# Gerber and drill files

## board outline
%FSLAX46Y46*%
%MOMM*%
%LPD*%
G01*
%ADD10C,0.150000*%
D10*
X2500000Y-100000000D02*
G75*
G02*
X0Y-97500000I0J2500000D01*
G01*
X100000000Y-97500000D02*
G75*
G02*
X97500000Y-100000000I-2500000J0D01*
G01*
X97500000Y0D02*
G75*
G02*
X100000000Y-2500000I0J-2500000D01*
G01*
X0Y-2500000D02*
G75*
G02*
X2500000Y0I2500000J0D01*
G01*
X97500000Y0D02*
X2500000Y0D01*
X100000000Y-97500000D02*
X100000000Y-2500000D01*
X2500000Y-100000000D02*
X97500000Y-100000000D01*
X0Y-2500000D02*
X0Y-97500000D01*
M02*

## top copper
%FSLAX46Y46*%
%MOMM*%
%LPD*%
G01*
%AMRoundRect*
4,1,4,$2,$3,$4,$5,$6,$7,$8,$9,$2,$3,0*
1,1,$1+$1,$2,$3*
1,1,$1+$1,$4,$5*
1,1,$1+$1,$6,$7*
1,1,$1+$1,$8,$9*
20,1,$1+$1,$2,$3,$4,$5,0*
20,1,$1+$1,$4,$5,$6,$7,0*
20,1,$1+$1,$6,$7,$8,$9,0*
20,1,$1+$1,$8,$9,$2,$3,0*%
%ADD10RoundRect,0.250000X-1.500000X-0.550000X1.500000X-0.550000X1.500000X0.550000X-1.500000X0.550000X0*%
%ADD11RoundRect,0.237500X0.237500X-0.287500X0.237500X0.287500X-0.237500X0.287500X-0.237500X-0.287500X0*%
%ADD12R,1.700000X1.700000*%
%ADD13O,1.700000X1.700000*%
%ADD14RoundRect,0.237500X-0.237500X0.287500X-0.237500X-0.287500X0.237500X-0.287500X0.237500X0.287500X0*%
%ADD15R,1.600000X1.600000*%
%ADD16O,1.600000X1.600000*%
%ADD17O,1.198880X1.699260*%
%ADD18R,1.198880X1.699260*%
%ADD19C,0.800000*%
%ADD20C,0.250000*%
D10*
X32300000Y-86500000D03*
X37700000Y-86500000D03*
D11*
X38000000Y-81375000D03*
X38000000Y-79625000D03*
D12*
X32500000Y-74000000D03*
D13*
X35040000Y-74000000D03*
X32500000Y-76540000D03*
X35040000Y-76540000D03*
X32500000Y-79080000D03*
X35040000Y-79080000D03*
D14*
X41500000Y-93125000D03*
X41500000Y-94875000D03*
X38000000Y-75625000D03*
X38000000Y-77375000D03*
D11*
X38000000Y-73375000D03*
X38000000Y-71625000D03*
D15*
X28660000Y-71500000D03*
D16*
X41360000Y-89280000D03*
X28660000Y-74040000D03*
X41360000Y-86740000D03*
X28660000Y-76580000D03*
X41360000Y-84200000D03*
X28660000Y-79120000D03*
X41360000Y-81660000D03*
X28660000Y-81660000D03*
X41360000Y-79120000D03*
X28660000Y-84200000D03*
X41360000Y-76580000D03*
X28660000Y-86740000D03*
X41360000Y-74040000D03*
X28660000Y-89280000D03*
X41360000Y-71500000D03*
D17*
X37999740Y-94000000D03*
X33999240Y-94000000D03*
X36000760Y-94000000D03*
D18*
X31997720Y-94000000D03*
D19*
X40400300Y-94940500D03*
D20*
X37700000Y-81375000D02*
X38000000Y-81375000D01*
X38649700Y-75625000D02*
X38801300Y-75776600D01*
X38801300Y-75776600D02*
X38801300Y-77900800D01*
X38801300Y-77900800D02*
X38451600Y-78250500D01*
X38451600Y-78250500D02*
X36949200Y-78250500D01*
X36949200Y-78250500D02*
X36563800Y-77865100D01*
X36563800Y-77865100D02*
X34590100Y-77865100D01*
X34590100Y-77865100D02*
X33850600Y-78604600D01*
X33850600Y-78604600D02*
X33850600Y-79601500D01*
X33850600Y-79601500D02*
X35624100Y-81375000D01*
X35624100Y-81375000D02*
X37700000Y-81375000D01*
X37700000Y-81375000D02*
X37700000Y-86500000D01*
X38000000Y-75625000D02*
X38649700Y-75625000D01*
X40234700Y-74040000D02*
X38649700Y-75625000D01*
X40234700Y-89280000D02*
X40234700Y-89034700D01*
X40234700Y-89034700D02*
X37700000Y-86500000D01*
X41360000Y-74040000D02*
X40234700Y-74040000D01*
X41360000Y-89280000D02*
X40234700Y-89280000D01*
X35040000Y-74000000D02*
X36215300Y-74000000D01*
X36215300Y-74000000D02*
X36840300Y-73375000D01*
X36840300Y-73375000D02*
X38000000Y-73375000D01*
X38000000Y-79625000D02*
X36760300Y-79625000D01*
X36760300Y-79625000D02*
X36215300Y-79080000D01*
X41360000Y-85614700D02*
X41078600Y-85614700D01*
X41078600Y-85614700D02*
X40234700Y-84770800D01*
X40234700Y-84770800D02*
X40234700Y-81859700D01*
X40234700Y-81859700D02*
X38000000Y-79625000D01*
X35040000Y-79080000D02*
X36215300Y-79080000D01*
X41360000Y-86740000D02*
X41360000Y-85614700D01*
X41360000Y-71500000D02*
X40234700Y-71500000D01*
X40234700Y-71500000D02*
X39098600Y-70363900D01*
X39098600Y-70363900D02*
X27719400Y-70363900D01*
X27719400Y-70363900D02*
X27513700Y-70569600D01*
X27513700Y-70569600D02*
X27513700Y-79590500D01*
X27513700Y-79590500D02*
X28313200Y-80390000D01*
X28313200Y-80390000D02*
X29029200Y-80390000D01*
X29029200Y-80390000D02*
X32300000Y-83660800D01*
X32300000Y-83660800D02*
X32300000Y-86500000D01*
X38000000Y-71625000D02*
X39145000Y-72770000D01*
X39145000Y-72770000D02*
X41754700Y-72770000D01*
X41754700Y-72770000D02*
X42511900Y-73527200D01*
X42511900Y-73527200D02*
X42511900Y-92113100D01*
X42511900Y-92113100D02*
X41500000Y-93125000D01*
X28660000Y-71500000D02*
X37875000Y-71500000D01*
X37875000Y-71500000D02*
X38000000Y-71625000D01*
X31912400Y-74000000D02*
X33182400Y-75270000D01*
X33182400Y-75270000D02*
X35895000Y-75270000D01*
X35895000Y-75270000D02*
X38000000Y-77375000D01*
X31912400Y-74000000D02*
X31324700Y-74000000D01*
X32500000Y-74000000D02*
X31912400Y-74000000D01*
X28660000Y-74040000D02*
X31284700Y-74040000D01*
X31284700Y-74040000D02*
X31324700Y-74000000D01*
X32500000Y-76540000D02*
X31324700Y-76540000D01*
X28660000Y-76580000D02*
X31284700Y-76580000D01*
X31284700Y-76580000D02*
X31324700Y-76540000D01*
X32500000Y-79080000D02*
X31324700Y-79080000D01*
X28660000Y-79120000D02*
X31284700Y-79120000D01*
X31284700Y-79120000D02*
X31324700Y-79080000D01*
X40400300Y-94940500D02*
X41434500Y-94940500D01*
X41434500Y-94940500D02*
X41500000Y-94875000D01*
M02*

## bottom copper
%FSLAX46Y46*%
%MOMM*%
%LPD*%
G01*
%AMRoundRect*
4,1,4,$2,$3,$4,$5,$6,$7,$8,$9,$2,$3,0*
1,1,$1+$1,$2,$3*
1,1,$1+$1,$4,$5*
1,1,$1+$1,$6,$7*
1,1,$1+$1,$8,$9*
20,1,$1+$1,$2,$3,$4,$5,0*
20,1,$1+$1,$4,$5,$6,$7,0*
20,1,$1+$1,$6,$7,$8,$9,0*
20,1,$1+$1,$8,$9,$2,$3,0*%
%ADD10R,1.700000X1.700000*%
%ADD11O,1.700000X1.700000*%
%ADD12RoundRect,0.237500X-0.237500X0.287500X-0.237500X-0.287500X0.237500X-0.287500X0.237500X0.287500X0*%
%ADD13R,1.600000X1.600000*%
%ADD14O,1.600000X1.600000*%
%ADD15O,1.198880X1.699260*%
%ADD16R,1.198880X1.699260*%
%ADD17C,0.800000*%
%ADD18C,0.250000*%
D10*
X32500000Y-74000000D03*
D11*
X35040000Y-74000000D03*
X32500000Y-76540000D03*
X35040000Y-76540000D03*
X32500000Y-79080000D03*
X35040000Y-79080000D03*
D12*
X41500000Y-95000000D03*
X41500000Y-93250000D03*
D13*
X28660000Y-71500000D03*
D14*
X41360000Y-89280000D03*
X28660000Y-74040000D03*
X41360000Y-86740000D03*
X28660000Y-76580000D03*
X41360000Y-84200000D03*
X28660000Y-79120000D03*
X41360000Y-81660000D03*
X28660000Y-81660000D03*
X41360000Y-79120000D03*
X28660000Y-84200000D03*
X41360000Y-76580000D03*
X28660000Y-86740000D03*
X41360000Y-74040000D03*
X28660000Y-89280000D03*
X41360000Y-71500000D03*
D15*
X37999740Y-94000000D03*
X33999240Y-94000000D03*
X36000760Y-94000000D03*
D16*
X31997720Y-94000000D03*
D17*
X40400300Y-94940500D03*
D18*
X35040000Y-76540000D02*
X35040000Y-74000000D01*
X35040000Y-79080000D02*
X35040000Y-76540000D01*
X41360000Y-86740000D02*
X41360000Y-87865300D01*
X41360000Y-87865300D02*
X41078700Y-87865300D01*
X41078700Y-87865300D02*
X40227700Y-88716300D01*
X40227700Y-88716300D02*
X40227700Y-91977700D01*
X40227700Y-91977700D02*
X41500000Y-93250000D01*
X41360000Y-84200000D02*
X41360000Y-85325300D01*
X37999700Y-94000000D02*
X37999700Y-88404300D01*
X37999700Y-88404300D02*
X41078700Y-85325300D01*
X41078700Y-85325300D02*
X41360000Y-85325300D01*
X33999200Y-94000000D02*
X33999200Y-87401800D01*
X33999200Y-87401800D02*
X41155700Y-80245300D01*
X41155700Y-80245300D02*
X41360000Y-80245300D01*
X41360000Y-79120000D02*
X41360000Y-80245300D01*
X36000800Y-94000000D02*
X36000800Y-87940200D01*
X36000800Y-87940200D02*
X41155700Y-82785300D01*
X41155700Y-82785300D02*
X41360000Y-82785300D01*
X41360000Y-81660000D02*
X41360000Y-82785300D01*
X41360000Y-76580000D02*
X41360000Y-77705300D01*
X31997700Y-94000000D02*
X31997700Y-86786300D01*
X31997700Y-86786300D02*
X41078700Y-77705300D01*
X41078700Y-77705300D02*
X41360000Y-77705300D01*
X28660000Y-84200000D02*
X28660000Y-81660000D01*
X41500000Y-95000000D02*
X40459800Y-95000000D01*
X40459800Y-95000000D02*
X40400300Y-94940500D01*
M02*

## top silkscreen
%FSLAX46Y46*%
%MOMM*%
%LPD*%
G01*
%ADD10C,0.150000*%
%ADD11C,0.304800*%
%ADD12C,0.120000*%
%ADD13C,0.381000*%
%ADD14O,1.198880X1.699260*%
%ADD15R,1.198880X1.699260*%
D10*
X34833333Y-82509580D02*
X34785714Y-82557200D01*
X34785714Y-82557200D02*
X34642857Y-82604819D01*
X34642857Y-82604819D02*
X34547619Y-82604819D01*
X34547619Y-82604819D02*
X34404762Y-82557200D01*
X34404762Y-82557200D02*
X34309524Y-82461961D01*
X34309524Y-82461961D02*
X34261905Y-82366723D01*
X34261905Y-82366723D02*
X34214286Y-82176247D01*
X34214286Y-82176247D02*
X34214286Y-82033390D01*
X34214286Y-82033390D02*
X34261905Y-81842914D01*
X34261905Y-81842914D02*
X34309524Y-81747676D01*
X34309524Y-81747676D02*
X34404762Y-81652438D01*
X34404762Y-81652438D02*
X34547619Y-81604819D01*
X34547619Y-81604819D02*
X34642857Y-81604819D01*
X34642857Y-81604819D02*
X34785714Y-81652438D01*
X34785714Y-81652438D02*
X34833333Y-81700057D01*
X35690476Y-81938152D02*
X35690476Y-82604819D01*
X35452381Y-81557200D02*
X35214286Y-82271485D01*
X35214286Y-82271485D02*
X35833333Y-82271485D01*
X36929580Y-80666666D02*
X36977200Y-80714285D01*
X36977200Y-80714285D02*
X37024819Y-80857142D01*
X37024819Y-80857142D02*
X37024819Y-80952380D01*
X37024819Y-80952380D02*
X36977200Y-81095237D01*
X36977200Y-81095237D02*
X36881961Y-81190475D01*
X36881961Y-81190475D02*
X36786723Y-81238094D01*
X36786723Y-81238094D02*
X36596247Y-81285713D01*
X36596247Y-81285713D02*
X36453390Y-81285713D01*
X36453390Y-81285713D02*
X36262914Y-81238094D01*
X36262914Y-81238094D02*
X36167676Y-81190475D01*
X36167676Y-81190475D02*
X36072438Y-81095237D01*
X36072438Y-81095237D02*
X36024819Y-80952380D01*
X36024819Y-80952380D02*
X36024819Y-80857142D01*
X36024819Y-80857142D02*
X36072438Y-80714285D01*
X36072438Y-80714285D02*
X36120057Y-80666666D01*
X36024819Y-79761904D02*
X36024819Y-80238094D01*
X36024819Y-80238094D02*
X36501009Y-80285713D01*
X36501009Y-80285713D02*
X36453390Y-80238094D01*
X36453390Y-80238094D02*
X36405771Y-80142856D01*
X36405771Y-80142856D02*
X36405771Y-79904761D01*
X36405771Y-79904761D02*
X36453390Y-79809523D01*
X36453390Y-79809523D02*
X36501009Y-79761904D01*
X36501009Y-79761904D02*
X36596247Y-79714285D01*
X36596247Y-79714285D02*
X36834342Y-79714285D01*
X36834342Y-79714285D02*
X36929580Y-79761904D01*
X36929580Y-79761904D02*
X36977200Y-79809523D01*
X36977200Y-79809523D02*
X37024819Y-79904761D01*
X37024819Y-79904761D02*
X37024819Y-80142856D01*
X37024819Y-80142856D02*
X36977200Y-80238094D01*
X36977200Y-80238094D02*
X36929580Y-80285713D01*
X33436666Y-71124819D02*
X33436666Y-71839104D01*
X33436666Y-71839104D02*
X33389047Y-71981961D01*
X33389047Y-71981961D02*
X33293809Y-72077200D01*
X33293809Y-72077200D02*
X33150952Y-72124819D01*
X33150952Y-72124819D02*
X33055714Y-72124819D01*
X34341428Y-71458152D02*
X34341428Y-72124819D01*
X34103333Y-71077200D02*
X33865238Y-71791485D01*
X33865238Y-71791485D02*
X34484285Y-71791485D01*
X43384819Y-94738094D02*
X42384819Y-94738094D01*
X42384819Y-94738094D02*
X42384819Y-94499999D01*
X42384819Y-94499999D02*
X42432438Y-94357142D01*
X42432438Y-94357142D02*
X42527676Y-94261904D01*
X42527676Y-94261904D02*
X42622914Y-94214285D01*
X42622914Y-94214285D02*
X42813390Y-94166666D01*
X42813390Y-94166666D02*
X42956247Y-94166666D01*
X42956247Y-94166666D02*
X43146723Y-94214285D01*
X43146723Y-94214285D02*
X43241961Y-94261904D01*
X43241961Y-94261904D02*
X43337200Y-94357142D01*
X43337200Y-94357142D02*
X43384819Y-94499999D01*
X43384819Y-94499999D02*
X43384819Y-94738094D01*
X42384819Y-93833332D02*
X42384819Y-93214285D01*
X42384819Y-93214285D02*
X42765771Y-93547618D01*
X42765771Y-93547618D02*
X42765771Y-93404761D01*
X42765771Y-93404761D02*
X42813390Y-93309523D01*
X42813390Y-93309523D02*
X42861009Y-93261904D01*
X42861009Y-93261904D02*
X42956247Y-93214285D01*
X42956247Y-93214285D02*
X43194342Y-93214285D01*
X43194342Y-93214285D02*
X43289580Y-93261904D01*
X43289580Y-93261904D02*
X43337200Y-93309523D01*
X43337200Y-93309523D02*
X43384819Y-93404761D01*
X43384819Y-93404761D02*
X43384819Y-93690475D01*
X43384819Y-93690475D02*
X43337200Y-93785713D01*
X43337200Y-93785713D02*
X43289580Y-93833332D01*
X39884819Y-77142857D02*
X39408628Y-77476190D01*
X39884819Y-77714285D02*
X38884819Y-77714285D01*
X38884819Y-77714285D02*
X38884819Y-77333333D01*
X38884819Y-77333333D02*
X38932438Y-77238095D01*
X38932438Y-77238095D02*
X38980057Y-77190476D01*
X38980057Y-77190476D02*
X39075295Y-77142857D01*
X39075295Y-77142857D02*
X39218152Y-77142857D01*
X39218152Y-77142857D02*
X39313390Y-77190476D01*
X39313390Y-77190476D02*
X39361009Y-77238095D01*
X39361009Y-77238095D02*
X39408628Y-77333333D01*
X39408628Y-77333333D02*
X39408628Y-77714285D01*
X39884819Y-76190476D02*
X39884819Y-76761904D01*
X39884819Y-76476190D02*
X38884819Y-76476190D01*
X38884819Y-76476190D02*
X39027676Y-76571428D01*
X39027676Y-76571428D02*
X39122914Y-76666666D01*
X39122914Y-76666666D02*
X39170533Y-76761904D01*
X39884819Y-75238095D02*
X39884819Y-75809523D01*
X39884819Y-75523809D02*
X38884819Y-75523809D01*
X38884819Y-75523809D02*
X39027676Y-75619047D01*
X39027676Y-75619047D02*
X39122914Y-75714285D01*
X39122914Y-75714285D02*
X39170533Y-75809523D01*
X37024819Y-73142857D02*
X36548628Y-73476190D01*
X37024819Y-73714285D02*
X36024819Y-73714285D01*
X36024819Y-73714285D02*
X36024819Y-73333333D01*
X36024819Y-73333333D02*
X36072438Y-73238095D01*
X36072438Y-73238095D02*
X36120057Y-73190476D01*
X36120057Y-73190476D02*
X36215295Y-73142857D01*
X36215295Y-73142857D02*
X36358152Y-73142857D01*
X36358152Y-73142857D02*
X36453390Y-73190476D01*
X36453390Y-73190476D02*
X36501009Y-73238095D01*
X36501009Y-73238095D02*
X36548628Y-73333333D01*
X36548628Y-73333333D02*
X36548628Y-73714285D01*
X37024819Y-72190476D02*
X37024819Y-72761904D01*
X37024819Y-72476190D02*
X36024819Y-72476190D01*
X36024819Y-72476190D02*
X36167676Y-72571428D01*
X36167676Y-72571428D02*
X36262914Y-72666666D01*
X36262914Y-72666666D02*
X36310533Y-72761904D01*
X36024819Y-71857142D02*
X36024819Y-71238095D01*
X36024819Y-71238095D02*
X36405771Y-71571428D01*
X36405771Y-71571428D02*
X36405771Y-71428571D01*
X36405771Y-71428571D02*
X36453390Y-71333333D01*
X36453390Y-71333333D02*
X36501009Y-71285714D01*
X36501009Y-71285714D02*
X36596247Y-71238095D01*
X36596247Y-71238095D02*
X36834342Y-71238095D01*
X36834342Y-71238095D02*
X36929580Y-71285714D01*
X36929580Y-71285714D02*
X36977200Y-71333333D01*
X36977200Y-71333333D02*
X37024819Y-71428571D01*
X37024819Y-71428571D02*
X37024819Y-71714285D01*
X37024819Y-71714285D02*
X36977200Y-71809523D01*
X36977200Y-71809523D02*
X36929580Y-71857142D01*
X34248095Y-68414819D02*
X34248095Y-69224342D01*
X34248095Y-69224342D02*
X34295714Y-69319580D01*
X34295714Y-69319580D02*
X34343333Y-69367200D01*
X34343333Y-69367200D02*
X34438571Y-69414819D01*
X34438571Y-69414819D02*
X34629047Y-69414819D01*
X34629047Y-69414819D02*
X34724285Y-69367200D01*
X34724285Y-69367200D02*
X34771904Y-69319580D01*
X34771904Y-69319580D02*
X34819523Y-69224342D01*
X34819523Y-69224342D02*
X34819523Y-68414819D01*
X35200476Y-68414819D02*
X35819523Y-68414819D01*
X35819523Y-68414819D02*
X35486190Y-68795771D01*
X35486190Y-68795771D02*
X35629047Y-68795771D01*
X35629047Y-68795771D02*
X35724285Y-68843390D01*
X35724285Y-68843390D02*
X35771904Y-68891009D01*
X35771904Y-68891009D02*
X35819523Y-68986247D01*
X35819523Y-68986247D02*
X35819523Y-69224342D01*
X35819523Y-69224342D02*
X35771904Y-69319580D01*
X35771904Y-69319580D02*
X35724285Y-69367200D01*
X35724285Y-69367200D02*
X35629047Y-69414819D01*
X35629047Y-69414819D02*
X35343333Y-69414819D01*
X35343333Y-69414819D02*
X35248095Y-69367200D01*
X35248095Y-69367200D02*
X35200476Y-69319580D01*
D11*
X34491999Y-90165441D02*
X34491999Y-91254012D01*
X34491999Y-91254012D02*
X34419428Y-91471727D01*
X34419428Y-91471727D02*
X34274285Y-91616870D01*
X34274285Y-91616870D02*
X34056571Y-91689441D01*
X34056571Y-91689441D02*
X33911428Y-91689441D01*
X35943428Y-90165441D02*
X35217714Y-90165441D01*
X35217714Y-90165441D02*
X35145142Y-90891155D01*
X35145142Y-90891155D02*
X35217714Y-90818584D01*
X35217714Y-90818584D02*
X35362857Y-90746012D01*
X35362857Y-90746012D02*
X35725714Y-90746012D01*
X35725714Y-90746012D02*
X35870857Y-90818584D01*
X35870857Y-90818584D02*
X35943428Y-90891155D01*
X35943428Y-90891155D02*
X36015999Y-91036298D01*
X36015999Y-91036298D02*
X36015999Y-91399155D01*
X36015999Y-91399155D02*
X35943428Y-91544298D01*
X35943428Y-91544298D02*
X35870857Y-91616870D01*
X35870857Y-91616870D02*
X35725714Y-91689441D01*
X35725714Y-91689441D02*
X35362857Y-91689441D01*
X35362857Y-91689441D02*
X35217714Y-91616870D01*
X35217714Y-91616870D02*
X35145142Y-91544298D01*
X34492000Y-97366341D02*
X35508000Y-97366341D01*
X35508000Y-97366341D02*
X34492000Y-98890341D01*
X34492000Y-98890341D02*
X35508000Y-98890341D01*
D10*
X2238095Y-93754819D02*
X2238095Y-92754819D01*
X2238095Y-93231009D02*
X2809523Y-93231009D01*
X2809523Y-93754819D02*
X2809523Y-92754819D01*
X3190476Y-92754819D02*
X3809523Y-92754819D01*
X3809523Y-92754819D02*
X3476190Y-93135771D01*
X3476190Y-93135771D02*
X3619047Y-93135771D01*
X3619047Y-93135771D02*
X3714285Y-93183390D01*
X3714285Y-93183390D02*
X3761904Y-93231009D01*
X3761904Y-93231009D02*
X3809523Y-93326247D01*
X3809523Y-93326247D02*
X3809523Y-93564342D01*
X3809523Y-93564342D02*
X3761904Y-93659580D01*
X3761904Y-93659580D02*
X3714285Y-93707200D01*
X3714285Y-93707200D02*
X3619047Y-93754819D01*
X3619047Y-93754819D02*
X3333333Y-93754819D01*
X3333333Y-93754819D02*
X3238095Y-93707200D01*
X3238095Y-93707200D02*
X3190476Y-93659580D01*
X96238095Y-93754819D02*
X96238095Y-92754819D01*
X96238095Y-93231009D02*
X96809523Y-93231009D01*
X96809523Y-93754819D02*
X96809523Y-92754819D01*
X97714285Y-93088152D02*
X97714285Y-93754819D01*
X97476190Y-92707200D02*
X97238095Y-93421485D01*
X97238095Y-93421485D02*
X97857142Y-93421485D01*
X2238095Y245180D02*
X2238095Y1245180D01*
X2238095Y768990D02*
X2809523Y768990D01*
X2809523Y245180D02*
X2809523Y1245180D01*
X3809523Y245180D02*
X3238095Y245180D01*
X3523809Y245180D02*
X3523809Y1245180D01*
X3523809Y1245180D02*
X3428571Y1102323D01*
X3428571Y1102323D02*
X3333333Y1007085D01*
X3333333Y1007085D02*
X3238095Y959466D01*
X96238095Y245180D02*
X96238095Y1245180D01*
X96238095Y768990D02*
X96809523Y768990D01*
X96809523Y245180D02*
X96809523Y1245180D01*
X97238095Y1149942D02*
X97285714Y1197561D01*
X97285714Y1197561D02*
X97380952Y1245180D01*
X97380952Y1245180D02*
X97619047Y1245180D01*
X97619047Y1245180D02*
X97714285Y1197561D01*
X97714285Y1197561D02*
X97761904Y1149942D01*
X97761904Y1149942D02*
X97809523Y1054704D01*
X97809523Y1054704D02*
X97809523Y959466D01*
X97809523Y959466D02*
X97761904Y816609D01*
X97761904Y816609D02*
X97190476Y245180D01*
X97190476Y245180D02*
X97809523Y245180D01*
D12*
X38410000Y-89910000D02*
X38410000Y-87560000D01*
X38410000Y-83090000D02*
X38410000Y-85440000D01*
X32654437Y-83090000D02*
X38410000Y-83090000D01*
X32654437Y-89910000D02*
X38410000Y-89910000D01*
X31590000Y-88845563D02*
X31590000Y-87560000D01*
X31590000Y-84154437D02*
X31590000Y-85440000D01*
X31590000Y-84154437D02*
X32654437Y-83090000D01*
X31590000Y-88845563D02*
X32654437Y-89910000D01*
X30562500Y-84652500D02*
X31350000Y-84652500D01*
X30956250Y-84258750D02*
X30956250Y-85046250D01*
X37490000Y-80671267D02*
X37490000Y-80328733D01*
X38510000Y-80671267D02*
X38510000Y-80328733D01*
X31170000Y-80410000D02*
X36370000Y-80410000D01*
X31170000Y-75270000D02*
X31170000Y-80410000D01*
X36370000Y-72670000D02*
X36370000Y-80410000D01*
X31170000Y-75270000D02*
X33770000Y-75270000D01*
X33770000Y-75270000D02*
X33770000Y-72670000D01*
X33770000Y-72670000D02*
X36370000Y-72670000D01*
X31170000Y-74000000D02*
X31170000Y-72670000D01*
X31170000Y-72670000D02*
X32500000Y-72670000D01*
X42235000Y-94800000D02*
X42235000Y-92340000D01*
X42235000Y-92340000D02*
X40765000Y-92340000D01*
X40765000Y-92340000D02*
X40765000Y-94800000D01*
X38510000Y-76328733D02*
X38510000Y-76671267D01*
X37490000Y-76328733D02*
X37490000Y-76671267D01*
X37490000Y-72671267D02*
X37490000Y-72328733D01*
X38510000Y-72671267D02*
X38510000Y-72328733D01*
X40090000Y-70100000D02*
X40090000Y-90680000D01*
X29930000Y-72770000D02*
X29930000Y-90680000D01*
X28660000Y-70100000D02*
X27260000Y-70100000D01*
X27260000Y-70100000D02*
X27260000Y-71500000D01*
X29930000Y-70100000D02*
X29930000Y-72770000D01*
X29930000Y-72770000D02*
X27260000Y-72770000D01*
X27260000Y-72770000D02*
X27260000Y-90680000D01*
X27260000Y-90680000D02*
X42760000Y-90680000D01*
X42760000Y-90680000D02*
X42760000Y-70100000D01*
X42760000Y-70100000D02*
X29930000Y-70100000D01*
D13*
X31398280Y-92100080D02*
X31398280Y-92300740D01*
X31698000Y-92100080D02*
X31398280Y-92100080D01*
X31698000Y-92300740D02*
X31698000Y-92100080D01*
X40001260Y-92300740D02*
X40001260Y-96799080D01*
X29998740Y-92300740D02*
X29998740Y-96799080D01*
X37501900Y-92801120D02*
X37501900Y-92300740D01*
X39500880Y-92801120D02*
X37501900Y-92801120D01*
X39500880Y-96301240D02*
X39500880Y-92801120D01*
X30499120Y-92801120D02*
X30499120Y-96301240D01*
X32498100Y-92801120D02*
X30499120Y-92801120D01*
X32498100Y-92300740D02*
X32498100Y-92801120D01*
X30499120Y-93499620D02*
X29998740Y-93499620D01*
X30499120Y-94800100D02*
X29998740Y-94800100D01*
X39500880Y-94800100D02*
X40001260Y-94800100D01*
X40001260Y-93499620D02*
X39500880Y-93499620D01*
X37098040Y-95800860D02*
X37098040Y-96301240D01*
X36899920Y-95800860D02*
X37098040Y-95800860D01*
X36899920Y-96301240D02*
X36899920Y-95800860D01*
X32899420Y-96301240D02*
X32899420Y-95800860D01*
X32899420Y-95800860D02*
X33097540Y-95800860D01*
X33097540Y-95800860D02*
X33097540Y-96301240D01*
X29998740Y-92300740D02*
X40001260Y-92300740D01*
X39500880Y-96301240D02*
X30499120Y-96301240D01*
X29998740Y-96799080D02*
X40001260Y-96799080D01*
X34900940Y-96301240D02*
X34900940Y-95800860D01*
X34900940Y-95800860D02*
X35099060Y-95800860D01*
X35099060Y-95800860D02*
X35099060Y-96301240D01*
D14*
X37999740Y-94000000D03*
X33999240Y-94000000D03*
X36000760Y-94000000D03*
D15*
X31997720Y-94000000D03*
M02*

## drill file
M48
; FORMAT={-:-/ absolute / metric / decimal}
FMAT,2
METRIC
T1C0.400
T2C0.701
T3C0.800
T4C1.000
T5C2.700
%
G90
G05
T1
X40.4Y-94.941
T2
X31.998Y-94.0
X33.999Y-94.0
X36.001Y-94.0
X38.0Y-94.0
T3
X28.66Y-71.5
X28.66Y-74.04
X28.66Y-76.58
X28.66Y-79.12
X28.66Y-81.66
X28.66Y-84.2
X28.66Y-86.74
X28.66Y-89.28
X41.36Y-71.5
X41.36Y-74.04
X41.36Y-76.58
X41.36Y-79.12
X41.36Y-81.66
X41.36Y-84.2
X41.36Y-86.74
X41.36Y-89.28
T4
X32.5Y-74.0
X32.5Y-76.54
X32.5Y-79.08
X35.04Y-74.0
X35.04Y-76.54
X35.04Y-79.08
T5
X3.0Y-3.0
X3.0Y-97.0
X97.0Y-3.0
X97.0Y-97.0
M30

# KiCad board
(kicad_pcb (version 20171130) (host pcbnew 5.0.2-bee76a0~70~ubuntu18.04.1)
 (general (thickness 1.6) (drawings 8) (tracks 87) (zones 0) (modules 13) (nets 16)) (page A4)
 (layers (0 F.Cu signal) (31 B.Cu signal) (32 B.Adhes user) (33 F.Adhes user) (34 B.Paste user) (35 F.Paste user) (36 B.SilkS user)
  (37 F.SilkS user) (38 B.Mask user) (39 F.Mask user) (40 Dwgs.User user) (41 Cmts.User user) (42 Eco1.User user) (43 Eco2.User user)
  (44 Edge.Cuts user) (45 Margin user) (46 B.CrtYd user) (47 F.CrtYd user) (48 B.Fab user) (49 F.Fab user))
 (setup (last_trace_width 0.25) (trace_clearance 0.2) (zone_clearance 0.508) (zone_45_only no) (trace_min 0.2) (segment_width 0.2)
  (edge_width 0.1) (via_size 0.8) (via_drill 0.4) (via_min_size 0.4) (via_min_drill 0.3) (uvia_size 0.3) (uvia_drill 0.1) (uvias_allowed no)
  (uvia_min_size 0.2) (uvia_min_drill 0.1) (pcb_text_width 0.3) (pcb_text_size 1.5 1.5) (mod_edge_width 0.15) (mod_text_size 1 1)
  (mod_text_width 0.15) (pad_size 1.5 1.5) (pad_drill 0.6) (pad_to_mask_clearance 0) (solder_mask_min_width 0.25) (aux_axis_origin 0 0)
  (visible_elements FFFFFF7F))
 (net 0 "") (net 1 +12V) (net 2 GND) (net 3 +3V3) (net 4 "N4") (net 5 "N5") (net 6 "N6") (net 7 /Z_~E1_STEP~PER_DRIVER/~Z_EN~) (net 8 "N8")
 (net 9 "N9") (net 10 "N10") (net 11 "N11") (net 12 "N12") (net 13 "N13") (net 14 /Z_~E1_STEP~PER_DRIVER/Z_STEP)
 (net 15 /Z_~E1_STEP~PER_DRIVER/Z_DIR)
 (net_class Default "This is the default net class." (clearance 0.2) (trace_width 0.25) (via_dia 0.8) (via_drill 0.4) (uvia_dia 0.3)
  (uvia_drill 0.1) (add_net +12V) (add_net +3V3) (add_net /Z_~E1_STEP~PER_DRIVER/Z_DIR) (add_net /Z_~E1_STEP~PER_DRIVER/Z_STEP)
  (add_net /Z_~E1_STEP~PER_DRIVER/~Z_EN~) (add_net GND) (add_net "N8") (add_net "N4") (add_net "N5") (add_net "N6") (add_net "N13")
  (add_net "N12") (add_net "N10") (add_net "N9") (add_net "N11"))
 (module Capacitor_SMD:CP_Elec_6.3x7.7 (layer F.Cu) (at 35 86.5)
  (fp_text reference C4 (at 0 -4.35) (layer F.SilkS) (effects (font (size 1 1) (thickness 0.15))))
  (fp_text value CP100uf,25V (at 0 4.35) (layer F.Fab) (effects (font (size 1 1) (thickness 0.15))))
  (fp_line (start 3.41 3.41) (end 3.41 1.06) (layer F.SilkS) (width 0.12))
  (fp_line (start 3.41 -3.41) (end 3.41 -1.06) (layer F.SilkS) (width 0.12))
  (fp_line (start -2.345563 -3.41) (end 3.41 -3.41) (layer F.SilkS) (width 0.12))
  (fp_line (start -2.345563 3.41) (end 3.41 3.41) (layer F.SilkS) (width 0.12))
  (fp_line (start -3.41 2.345563) (end -3.41 1.06) (layer F.SilkS) (width 0.12))
  (fp_line (start -3.41 -2.345563) (end -3.41 -1.06) (layer F.SilkS) (width 0.12))
  (fp_line (start -3.41 -2.345563) (end -2.345563 -3.41) (layer F.SilkS) (width 0.12))
  (fp_line (start -3.41 2.345563) (end -2.345563 3.41) (layer F.SilkS) (width 0.12))
  (fp_line (start -4.4375 -1.8475) (end -3.65 -1.8475) (layer F.SilkS) (width 0.12))
  (fp_line (start -4.04375 -2.24125) (end -4.04375 -1.45375) (layer F.SilkS) (width 0.12))
  (pad 1 smd roundrect (at -2.7 0) (size 3.5 1.6) (layers F.Cu F.Paste F.Mask) (roundrect_rratio 0.15625) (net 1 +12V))
  (pad 2 smd roundrect (at 2.7 0) (size 3.5 1.6) (layers F.Cu F.Paste F.Mask) (roundrect_rratio 0.15625) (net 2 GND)))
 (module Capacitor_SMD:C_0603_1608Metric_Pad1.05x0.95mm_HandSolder (layer F.Cu) (at 38 80.5 90)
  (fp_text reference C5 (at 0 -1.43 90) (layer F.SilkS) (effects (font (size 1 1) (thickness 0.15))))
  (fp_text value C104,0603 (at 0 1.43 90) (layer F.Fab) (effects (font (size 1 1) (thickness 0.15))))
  (fp_line (start -0.171267 -0.51) (end 0.171267 -0.51) (layer F.SilkS) (width 0.12))
  (fp_line (start -0.171267 0.51) (end 0.171267 0.51) (layer F.SilkS) (width 0.12))
  (pad 1 smd roundrect (at -0.875 0 90) (size 1.05 0.95) (layers F.Cu F.Paste F.Mask) (roundrect_rratio 0.25) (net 2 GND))
  (pad 2 smd roundrect (at 0.875 0 90) (size 1.05 0.95) (layers F.Cu F.Paste F.Mask) (roundrect_rratio 0.25) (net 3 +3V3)))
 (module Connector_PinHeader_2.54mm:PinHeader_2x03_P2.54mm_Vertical (layer F.Cu) (at 32.5 74)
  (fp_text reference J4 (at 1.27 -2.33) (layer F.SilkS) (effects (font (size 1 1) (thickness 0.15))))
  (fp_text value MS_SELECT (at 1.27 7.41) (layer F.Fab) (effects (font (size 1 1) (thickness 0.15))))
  (fp_line (start -1.33 6.41) (end 3.87 6.41) (layer F.SilkS) (width 0.12))
  (fp_line (start -1.33 1.27) (end -1.33 6.41) (layer F.SilkS) (width 0.12))
  (fp_line (start 3.87 -1.33) (end 3.87 6.41) (layer F.SilkS) (width 0.12))
  (fp_line (start -1.33 1.27) (end 1.27 1.27) (layer F.SilkS) (width 0.12))
  (fp_line (start 1.27 1.27) (end 1.27 -1.33) (layer F.SilkS) (width 0.12))
  (fp_line (start 1.27 -1.33) (end 3.87 -1.33) (layer F.SilkS) (width 0.12))
  (fp_line (start -1.33 0) (end -1.33 -1.33) (layer F.SilkS) (width 0.12))
  (fp_line (start -1.33 -1.33) (end 0 -1.33) (layer F.SilkS) (width 0.12))
  (pad 1 thru_hole rect (at 0 0) (size 1.7 1.7) (drill 1) (layers *.Cu *.Mask) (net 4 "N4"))
  (pad 2 thru_hole oval (at 2.54 0) (size 1.7 1.7) (drill 1) (layers *.Cu *.Mask) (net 3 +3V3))
  (pad 3 thru_hole oval (at 0 2.54) (size 1.7 1.7) (drill 1) (layers *.Cu *.Mask) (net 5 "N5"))
  (pad 4 thru_hole oval (at 2.54 2.54) (size 1.7 1.7) (drill 1) (layers *.Cu *.Mask) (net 3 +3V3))
  (pad 5 thru_hole oval (at 0 5.08) (size 1.7 1.7) (drill 1) (layers *.Cu *.Mask) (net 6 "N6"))
  (pad 6 thru_hole oval (at 2.54 5.08) (size 1.7 1.7) (drill 1) (layers *.Cu *.Mask) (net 3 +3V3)))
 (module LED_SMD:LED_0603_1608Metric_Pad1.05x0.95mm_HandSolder (layer F.Cu) (at 41.5 94 270)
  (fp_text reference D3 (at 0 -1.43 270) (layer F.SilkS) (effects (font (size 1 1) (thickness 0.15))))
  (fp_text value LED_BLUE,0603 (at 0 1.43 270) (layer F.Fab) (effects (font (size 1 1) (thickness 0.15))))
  (fp_line (start 0.8 -0.735) (end -1.66 -0.735) (layer F.SilkS) (width 0.12))
  (fp_line (start -1.66 -0.735) (end -1.66 0.735) (layer F.SilkS) (width 0.12))
  (fp_line (start -1.66 0.735) (end 0.8 0.735) (layer F.SilkS) (width 0.12))
  (pad 1 smd roundrect (at -0.875 0 270) (size 1.05 0.95) (layers F.Cu F.Paste F.Mask) (roundrect_rratio 0.25)
   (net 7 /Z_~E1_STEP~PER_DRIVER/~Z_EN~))
  (pad 2 smd roundrect (at 0.875 0 270) (size 1.05 0.95) (layers F.Cu F.Paste F.Mask) (roundrect_rratio 0.25) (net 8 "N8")))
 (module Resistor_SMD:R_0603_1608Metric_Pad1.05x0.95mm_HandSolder (layer F.Cu) (at 38 76.5 270)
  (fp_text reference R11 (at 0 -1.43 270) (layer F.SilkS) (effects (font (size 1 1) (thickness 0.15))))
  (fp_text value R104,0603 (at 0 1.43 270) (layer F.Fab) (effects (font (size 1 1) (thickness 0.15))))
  (fp_line (start -0.171267 -0.51) (end 0.171267 -0.51) (layer F.SilkS) (width 0.12))
  (fp_line (start -0.171267 0.51) (end 0.171267 0.51) (layer F.SilkS) (width 0.12))
  (pad 1 smd roundrect (at -0.875 0 270) (size 1.05 0.95) (layers F.Cu F.Paste F.Mask) (roundrect_rratio 0.25) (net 2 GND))
  (pad 2 smd roundrect (at 0.875 0 270) (size 1.05 0.95) (layers F.Cu F.Paste F.Mask) (roundrect_rratio 0.25) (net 4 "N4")))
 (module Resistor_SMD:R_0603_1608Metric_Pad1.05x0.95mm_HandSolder (layer B.Cu) (at 41.5 94.125 270)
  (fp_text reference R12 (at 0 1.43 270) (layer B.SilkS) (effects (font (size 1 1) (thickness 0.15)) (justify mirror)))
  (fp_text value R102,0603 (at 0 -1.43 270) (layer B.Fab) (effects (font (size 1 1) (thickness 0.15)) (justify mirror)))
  (pad 2 smd roundrect (at 0.875 0 270) (size 1.05 0.95) (layers B.Cu B.Paste B.Mask) (roundrect_rratio 0.25) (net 8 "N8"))
  (pad 1 smd roundrect (at -0.875 0 270) (size 1.05 0.95) (layers B.Cu B.Paste B.Mask) (roundrect_rratio 0.25) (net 3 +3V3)))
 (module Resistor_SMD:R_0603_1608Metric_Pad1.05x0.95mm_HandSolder (layer F.Cu) (at 38 72.5 90)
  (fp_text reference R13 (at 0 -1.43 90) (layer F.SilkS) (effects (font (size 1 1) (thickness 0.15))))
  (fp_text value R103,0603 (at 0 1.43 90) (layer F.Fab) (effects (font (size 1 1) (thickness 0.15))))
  (fp_line (start -0.171267 -0.51) (end 0.171267 -0.51) (layer F.SilkS) (width 0.12))
  (fp_line (start -0.171267 0.51) (end 0.171267 0.51) (layer F.SilkS) (width 0.12))
  (pad 1 smd roundrect (at -0.875 0 90) (size 1.05 0.95) (layers F.Cu F.Paste F.Mask) (roundrect_rratio 0.25) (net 3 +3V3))
  (pad 2 smd roundrect (at 0.875 0 90) (size 1.05 0.95) (layers F.Cu F.Paste F.Mask) (roundrect_rratio 0.25)
   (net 7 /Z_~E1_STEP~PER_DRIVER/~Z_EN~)))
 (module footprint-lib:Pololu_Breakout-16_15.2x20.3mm (layer F.Cu) (at 28.66 71.5)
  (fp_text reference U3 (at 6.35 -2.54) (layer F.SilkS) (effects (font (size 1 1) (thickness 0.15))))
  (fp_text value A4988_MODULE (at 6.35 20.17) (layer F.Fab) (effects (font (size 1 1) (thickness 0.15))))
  (fp_line (start 11.43 -1.4) (end 11.43 19.18) (layer F.SilkS) (width 0.12))
  (fp_line (start 1.27 1.27) (end 1.27 19.18) (layer F.SilkS) (width 0.12))
  (fp_line (start 0 -1.4) (end -1.4 -1.4) (layer F.SilkS) (width 0.12))
  (fp_line (start -1.4 -1.4) (end -1.4 0) (layer F.SilkS) (width 0.12))
  (fp_line (start 1.27 -1.4) (end 1.27 1.27) (layer F.SilkS) (width 0.12))
  (fp_line (start 1.27 1.27) (end -1.4 1.27) (layer F.SilkS) (width 0.12))
  (fp_line (start -1.4 1.27) (end -1.4 19.18) (layer F.SilkS) (width 0.12))
  (fp_line (start -1.4 19.18) (end 14.1 19.18) (layer F.SilkS) (width 0.12))
  (fp_line (start 14.1 19.18) (end 14.1 -1.4) (layer F.SilkS) (width 0.12))
  (fp_line (start 14.1 -1.4) (end 1.27 -1.4) (layer F.SilkS) (width 0.12))
  (pad 1 thru_hole rect (at 0 0) (size 1.6 1.6) (drill 0.8) (layers *.Cu *.Mask) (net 7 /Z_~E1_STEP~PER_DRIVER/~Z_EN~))
  (pad 9 thru_hole oval (at 12.7 17.78) (size 1.6 1.6) (drill 0.8) (layers *.Cu *.Mask) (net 2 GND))
  (pad 2 thru_hole oval (at 0 2.54) (size 1.6 1.6) (drill 0.8) (layers *.Cu *.Mask) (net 4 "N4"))
  (pad 10 thru_hole oval (at 12.7 15.24) (size 1.6 1.6) (drill 0.8) (layers *.Cu *.Mask) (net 3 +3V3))
  (pad 3 thru_hole oval (at 0 5.08) (size 1.6 1.6) (drill 0.8) (layers *.Cu *.Mask) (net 5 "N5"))
  (pad 11 thru_hole oval (at 12.7 12.7) (size 1.6 1.6) (drill 0.8) (layers *.Cu *.Mask) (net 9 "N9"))
  (pad 4 thru_hole oval (at 0 7.62) (size 1.6 1.6) (drill 0.8) (layers *.Cu *.Mask) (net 6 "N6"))
  (pad 12 thru_hole oval (at 12.7 10.16) (size 1.6 1.6) (drill 0.8) (layers *.Cu *.Mask) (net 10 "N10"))
  (pad 5 thru_hole oval (at 0 10.16) (size 1.6 1.6) (drill 0.8) (layers *.Cu *.Mask) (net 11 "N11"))
  (pad 13 thru_hole oval (at 12.7 7.62) (size 1.6 1.6) (drill 0.8) (layers *.Cu *.Mask) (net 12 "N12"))
  (pad 6 thru_hole oval (at 0 12.7) (size 1.6 1.6) (drill 0.8) (layers *.Cu *.Mask) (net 11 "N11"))
  (pad 14 thru_hole oval (at 12.7 5.08) (size 1.6 1.6) (drill 0.8) (layers *.Cu *.Mask) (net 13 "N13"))
  (pad 7 thru_hole oval (at 0 15.24) (size 1.6 1.6) (drill 0.8) (layers *.Cu *.Mask) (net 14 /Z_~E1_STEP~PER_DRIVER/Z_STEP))
  (pad 15 thru_hole oval (at 12.7 2.54) (size 1.6 1.6) (drill 0.8) (layers *.Cu *.Mask) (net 2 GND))
  (pad 8 thru_hole oval (at 0 17.78) (size 1.6 1.6) (drill 0.8) (layers *.Cu *.Mask) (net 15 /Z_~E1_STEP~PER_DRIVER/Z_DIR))
  (pad 16 thru_hole oval (at 12.7 0) (size 1.6 1.6) (drill 0.8) (layers *.Cu *.Mask) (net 1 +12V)))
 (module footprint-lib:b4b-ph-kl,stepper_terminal (layer F.Cu) (at 35 94)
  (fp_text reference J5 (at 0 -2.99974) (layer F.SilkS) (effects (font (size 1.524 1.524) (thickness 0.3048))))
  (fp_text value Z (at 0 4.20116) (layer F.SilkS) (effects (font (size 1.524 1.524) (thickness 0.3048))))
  (fp_line (start -3.60172 -1.89992) (end -3.60172 -1.69926) (layer F.SilkS) (width 0.381))
  (fp_line (start -3.302 -1.89992) (end -3.60172 -1.89992) (layer F.SilkS) (width 0.381))
  (fp_line (start -3.302 -1.69926) (end -3.302 -1.89992) (layer F.SilkS) (width 0.381))
  (fp_line (start 5.00126 -1.69926) (end 5.00126 2.79908) (layer F.SilkS) (width 0.381))
  (fp_line (start -5.00126 -1.69926) (end -5.00126 2.79908) (layer F.SilkS) (width 0.381))
  (fp_line (start 2.5019 -1.19888) (end 2.5019 -1.69926) (layer F.SilkS) (width 0.381))
  (fp_line (start 4.50088 -1.19888) (end 2.5019 -1.19888) (layer F.SilkS) (width 0.381))
  (fp_line (start 4.50088 2.30124) (end 4.50088 -1.19888) (layer F.SilkS) (width 0.381))
  (fp_line (start -4.50088 -1.19888) (end -4.50088 2.30124) (layer F.SilkS) (width 0.381))
  (fp_line (start -2.5019 -1.19888) (end -4.50088 -1.19888) (layer F.SilkS) (width 0.381))
  (fp_line (start -2.5019 -1.69926) (end -2.5019 -1.19888) (layer F.SilkS) (width 0.381))
  (fp_line (start -4.50088 -0.50038) (end -5.00126 -0.50038) (layer F.SilkS) (width 0.381))
  (fp_line (start -4.50088 0.8001) (end -5.00126 0.8001) (layer F.SilkS) (width 0.381))
  (fp_line (start 4.50088 0.8001) (end 5.00126 0.8001) (layer F.SilkS) (width 0.381))
  (fp_line (start 5.00126 -0.50038) (end 4.50088 -0.50038) (layer F.SilkS) (width 0.381))
  (fp_line (start 2.09804 1.80086) (end 2.09804 2.30124) (layer F.SilkS) (width 0.381))
  (fp_line (start 1.89992 1.80086) (end 2.09804 1.80086) (layer F.SilkS) (width 0.381))
  (fp_line (start 1.89992 2.30124) (end 1.89992 1.80086) (layer F.SilkS) (width 0.381))
  (fp_line (start -2.10058 2.30124) (end -2.10058 1.80086) (layer F.SilkS) (width 0.381))
  (fp_line (start -2.10058 1.80086) (end -1.90246 1.80086) (layer F.SilkS) (width 0.381))
  (fp_line (start -1.90246 1.80086) (end -1.90246 2.30124) (layer F.SilkS) (width 0.381))
  (fp_line (start -5.00126 -1.69926) (end 5.00126 -1.69926) (layer F.SilkS) (width 0.381))
  (fp_line (start 4.50088 2.30124) (end -4.50088 2.30124) (layer F.SilkS) (width 0.381))
  (fp_line (start -5.00126 2.79908) (end 5.00126 2.79908) (layer F.SilkS) (width 0.381))
  (fp_line (start -0.09906 2.30124) (end -0.09906 1.80086) (layer F.SilkS) (width 0.381))
  (fp_line (start -0.09906 1.80086) (end 0.09906 1.80086) (layer F.SilkS) (width 0.381))
  (fp_line (start 0.09906 1.80086) (end 0.09906 2.30124) (layer F.SilkS) (width 0.381))
  (pad 4 thru_hole oval (at 2.99974 0) (size 1.19888 1.69926) (drill 0.70104) (layers *.Cu *.Mask F.SilkS) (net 9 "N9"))
  (pad 2 thru_hole oval (at -1.00076 0) (size 1.19888 1.69926) (drill 0.70104) (layers *.Cu *.Mask F.SilkS) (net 12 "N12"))
  (pad 3 thru_hole oval (at 1.00076 0) (size 1.19888 1.69926) (drill 0.70104) (layers *.Cu *.Mask F.SilkS) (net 10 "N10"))
  (pad 1 thru_hole rect (at -3.00228 0) (size 1.19888 1.69926) (drill 0.70104) (layers *.Cu *.Mask F.SilkS) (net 13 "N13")))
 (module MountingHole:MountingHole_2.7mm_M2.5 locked (layer F.Cu) (at 3 97)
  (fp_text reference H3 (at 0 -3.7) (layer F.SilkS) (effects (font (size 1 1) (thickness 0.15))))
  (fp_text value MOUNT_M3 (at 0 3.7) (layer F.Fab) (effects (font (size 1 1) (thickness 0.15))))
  (pad 1 np_thru_hole circle (at 0 0) (size 2.7 2.7) (drill 2.7) (layers *.Cu *.Mask)))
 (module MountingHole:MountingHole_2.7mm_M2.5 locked (layer F.Cu) (at 97 97)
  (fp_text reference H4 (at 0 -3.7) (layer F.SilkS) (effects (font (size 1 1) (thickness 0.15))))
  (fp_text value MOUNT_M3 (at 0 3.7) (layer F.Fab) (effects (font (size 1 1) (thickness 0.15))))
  (pad 1 np_thru_hole circle (at 0 0) (size 2.7 2.7) (drill 2.7) (layers *.Cu *.Mask)))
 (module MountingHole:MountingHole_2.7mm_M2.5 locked (layer F.Cu) (at 3 3)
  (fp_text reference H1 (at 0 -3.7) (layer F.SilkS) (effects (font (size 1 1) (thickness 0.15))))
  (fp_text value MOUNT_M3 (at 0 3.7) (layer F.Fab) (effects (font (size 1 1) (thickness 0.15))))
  (pad 1 np_thru_hole circle (at 0 0) (size 2.7 2.7) (drill 2.7) (layers *.Cu *.Mask)))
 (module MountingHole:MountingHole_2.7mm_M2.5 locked (layer F.Cu) (at 97 3)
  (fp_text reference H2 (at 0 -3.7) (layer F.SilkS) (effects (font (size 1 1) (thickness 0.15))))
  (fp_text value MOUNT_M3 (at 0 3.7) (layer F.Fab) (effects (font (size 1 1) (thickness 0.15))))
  (pad 1 np_thru_hole circle (at 0 0) (size 2.7 2.7) (drill 2.7) (layers *.Cu *.Mask)))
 (gr_arc (start 2.5 97.5) (end 0 97.5) (angle -90) (layer Edge.Cuts) (width 0.15))
 (gr_arc (start 97.5 97.5) (end 97.5 100) (angle -90) (layer Edge.Cuts) (width 0.15))
 (gr_arc (start 97.5 2.5) (end 100 2.5) (angle -90) (layer Edge.Cuts) (width 0.15))
 (gr_arc (start 2.5 2.5) (end 2.5 0) (angle -90) (layer Edge.Cuts) (width 0.15))
 (gr_line (start 97.5 0) (end 2.5 0) (layer Edge.Cuts) (width 0.15))
 (gr_line (start 100 97.5) (end 100 2.5) (layer Edge.Cuts) (width 0.15))
 (gr_line (start 2.5 100) (end 97.5 100) (layer Edge.Cuts) (width 0.15))
 (gr_line (start 0 2.5) (end 0 97.5) (layer Edge.Cuts) (width 0.15))
 (segment (start 37.7 81.375) (end 38 81.375) (width 0.25) (layer F.Cu) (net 2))
 (segment (start 38.6497 75.625) (end 38.8013 75.7766) (width 0.25) (layer F.Cu) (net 2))
 (segment (start 38.8013 75.7766) (end 38.8013 77.9008) (width 0.25) (layer F.Cu) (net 2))
 (segment (start 38.8013 77.9008) (end 38.4516 78.2505) (width 0.25) (layer F.Cu) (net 2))
 (segment (start 38.4516 78.2505) (end 36.9492 78.2505) (width 0.25) (layer F.Cu) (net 2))
 (segment (start 36.9492 78.2505) (end 36.5638 77.8651) (width 0.25) (layer F.Cu) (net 2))
 (segment (start 36.5638 77.8651) (end 34.5901 77.8651) (width 0.25) (layer F.Cu) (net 2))
 (segment (start 34.5901 77.8651) (end 33.8506 78.6046) (width 0.25) (layer F.Cu) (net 2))
 (segment (start 33.8506 78.6046) (end 33.8506 79.6015) (width 0.25) (layer F.Cu) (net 2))
 (segment (start 33.8506 79.6015) (end 35.6241 81.375) (width 0.25) (layer F.Cu) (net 2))
 (segment (start 35.6241 81.375) (end 37.7 81.375) (width 0.25) (layer F.Cu) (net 2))
 (segment (start 37.7 81.375) (end 37.7 86.5) (width 0.25) (layer F.Cu) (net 2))
 (segment (start 38 75.625) (end 38.6497 75.625) (width 0.25) (layer F.Cu) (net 2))
 (segment (start 40.2347 74.04) (end 38.6497 75.625) (width 0.25) (layer F.Cu) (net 2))
 (segment (start 40.2347 89.28) (end 40.2347 89.0347) (width 0.25) (layer F.Cu) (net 2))
 (segment (start 40.2347 89.0347) (end 37.7 86.5) (width 0.25) (layer F.Cu) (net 2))
 (segment (start 41.36 74.04) (end 40.2347 74.04) (width 0.25) (layer F.Cu) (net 2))
 (segment (start 41.36 89.28) (end 40.2347 89.28) (width 0.25) (layer F.Cu) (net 2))
 (segment (start 35.04 74) (end 36.2153 74) (width 0.25) (layer F.Cu) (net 3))
 (segment (start 36.2153 74) (end 36.8403 73.375) (width 0.25) (layer F.Cu) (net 3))
 (segment (start 36.8403 73.375) (end 38 73.375) (width 0.25) (layer F.Cu) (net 3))
 (segment (start 38 79.625) (end 36.7603 79.625) (width 0.25) (layer F.Cu) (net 3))
 (segment (start 36.7603 79.625) (end 36.2153 79.08) (width 0.25) (layer F.Cu) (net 3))
 (segment (start 41.36 85.6147) (end 41.0786 85.6147) (width 0.25) (layer F.Cu) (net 3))
 (segment (start 41.0786 85.6147) (end 40.2347 84.7708) (width 0.25) (layer F.Cu) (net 3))
 (segment (start 40.2347 84.7708) (end 40.2347 81.8597) (width 0.25) (layer F.Cu) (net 3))
 (segment (start 40.2347 81.8597) (end 38 79.625) (width 0.25) (layer F.Cu) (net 3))
 (segment (start 35.04 79.08) (end 36.2153 79.08) (width 0.25) (layer F.Cu) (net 3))
 (segment (start 35.04 76.54) (end 35.04 74) (width 0.25) (layer B.Cu) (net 3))
 (segment (start 35.04 79.08) (end 35.04 76.54) (width 0.25) (layer B.Cu) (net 3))
 (segment (start 41.36 86.74) (end 41.36 85.6147) (width 0.25) (layer F.Cu) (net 3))
 (segment (start 41.36 86.74) (end 41.36 87.8653) (width 0.25) (layer B.Cu) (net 3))
 (segment (start 41.36 87.8653) (end 41.0787 87.8653) (width 0.25) (layer B.Cu) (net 3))
 (segment (start 41.0787 87.8653) (end 40.2277 88.7163) (width 0.25) (layer B.Cu) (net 3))
 (segment (start 40.2277 88.7163) (end 40.2277 91.9777) (width 0.25) (layer B.Cu) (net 3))
 (segment (start 40.2277 91.9777) (end 41.5 93.25) (width 0.25) (layer B.Cu) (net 3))
 (segment (start 41.36 71.5) (end 40.2347 71.5) (width 0.25) (layer F.Cu) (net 1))
 (segment (start 40.2347 71.5) (end 39.0986 70.3639) (width 0.25) (layer F.Cu) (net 1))
 (segment (start 39.0986 70.3639) (end 27.7194 70.3639) (width 0.25) (layer F.Cu) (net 1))
 (segment (start 27.7194 70.3639) (end 27.5137 70.5696) (width 0.25) (layer F.Cu) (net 1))
 (segment (start 27.5137 70.5696) (end 27.5137 79.5905) (width 0.25) (layer F.Cu) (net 1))
 (segment (start 27.5137 79.5905) (end 28.3132 80.39) (width 0.25) (layer F.Cu) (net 1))
 (segment (start 28.3132 80.39) (end 29.0292 80.39) (width 0.25) (layer F.Cu) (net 1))
 (segment (start 29.0292 80.39) (end 32.3 83.6608) (width 0.25) (layer F.Cu) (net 1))
 (segment (start 32.3 83.6608) (end 32.3 86.5) (width 0.25) (layer F.Cu) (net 1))
 (segment (start 41.36 84.2) (end 41.36 85.3253) (width 0.25) (layer B.Cu) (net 9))
 (segment (start 37.9997 94) (end 37.9997 88.4043) (width 0.25) (layer B.Cu) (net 9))
 (segment (start 37.9997 88.4043) (end 41.0787 85.3253) (width 0.25) (layer B.Cu) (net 9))
 (segment (start 41.0787 85.3253) (end 41.36 85.3253) (width 0.25) (layer B.Cu) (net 9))
 (segment (start 33.9992 94) (end 33.9992 87.4018) (width 0.25) (layer B.Cu) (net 12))
 (segment (start 33.9992 87.4018) (end 41.1557 80.2453) (width 0.25) (layer B.Cu) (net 12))
 (segment (start 41.1557 80.2453) (end 41.36 80.2453) (width 0.25) (layer B.Cu) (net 12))
 (segment (start 41.36 79.12) (end 41.36 80.2453) (width 0.25) (layer B.Cu) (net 12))
 (segment (start 36.0008 94) (end 36.0008 87.9402) (width 0.25) (layer B.Cu) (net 10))
 (segment (start 36.0008 87.9402) (end 41.1557 82.7853) (width 0.25) (layer B.Cu) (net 10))
 (segment (start 41.1557 82.7853) (end 41.36 82.7853) (width 0.25) (layer B.Cu) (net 10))
 (segment (start 41.36 81.66) (end 41.36 82.7853) (width 0.25) (layer B.Cu) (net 10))
 (segment (start 41.36 76.58) (end 41.36 77.7053) (width 0.25) (layer B.Cu) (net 13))
 (segment (start 31.9977 94) (end 31.9977 86.7863) (width 0.25) (layer B.Cu) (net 13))
 (segment (start 31.9977 86.7863) (end 41.0787 77.7053) (width 0.25) (layer B.Cu) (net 13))
 (segment (start 41.0787 77.7053) (end 41.36 77.7053) (width 0.25) (layer B.Cu) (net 13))
 (segment (start 38 71.625) (end 39.145 72.77) (width 0.25) (layer F.Cu) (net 7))
 (segment (start 39.145 72.77) (end 41.7547 72.77) (width 0.25) (layer F.Cu) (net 7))
 (segment (start 41.7547 72.77) (end 42.5119 73.5272) (width 0.25) (layer F.Cu) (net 7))
 (segment (start 42.5119 73.5272) (end 42.5119 92.1131) (width 0.25) (layer F.Cu) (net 7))
 (segment (start 42.5119 92.1131) (end 41.5 93.125) (width 0.25) (layer F.Cu) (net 7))
 (segment (start 28.66 71.5) (end 37.875 71.5) (width 0.25) (layer F.Cu) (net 7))
 (segment (start 37.875 71.5) (end 38 71.625) (width 0.25) (layer F.Cu) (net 7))
 (segment (start 31.9124 74) (end 33.1824 75.27) (width 0.25) (layer F.Cu) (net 4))
 (segment (start 33.1824 75.27) (end 35.895 75.27) (width 0.25) (layer F.Cu) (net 4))
 (segment (start 35.895 75.27) (end 38 77.375) (width 0.25) (layer F.Cu) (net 4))
 (segment (start 31.9124 74) (end 31.3247 74) (width 0.25) (layer F.Cu) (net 4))
 (segment (start 32.5 74) (end 31.9124 74) (width 0.25) (layer F.Cu) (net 4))
 (segment (start 28.66 74.04) (end 31.2847 74.04) (width 0.25) (layer F.Cu) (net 4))
 (segment (start 31.2847 74.04) (end 31.3247 74) (width 0.25) (layer F.Cu) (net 4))
 (segment (start 32.5 76.54) (end 31.3247 76.54) (width 0.25) (layer F.Cu) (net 5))
 (segment (start 28.66 76.58) (end 31.2847 76.58) (width 0.25) (layer F.Cu) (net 5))
 (segment (start 31.2847 76.58) (end 31.3247 76.54) (width 0.25) (layer F.Cu) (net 5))
 (segment (start 32.5 79.08) (end 31.3247 79.08) (width 0.25) (layer F.Cu) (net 6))
 (segment (start 28.66 79.12) (end 31.2847 79.12) (width 0.25) (layer F.Cu) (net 6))
 (segment (start 31.2847 79.12) (end 31.3247 79.08) (width 0.25) (layer F.Cu) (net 6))
 (segment (start 28.66 84.2) (end 28.66 81.66) (width 0.25) (layer B.Cu) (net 11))
 (segment (start 40.4003 94.9405) (end 41.4345 94.9405) (width 0.25) (layer F.Cu) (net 8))
 (segment (start 41.4345 94.9405) (end 41.5 94.875) (width 0.25) (layer F.Cu) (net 8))
 (segment (start 41.5 95) (end 40.4598 95) (width 0.25) (layer B.Cu) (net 8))
 (segment (start 40.4598 95) (end 40.4003 94.9405) (width 0.25) (layer B.Cu) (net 8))
 (via (at 40.4003 94.9405) (size 0.8) (layers F.Cu B.Cu) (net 8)))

